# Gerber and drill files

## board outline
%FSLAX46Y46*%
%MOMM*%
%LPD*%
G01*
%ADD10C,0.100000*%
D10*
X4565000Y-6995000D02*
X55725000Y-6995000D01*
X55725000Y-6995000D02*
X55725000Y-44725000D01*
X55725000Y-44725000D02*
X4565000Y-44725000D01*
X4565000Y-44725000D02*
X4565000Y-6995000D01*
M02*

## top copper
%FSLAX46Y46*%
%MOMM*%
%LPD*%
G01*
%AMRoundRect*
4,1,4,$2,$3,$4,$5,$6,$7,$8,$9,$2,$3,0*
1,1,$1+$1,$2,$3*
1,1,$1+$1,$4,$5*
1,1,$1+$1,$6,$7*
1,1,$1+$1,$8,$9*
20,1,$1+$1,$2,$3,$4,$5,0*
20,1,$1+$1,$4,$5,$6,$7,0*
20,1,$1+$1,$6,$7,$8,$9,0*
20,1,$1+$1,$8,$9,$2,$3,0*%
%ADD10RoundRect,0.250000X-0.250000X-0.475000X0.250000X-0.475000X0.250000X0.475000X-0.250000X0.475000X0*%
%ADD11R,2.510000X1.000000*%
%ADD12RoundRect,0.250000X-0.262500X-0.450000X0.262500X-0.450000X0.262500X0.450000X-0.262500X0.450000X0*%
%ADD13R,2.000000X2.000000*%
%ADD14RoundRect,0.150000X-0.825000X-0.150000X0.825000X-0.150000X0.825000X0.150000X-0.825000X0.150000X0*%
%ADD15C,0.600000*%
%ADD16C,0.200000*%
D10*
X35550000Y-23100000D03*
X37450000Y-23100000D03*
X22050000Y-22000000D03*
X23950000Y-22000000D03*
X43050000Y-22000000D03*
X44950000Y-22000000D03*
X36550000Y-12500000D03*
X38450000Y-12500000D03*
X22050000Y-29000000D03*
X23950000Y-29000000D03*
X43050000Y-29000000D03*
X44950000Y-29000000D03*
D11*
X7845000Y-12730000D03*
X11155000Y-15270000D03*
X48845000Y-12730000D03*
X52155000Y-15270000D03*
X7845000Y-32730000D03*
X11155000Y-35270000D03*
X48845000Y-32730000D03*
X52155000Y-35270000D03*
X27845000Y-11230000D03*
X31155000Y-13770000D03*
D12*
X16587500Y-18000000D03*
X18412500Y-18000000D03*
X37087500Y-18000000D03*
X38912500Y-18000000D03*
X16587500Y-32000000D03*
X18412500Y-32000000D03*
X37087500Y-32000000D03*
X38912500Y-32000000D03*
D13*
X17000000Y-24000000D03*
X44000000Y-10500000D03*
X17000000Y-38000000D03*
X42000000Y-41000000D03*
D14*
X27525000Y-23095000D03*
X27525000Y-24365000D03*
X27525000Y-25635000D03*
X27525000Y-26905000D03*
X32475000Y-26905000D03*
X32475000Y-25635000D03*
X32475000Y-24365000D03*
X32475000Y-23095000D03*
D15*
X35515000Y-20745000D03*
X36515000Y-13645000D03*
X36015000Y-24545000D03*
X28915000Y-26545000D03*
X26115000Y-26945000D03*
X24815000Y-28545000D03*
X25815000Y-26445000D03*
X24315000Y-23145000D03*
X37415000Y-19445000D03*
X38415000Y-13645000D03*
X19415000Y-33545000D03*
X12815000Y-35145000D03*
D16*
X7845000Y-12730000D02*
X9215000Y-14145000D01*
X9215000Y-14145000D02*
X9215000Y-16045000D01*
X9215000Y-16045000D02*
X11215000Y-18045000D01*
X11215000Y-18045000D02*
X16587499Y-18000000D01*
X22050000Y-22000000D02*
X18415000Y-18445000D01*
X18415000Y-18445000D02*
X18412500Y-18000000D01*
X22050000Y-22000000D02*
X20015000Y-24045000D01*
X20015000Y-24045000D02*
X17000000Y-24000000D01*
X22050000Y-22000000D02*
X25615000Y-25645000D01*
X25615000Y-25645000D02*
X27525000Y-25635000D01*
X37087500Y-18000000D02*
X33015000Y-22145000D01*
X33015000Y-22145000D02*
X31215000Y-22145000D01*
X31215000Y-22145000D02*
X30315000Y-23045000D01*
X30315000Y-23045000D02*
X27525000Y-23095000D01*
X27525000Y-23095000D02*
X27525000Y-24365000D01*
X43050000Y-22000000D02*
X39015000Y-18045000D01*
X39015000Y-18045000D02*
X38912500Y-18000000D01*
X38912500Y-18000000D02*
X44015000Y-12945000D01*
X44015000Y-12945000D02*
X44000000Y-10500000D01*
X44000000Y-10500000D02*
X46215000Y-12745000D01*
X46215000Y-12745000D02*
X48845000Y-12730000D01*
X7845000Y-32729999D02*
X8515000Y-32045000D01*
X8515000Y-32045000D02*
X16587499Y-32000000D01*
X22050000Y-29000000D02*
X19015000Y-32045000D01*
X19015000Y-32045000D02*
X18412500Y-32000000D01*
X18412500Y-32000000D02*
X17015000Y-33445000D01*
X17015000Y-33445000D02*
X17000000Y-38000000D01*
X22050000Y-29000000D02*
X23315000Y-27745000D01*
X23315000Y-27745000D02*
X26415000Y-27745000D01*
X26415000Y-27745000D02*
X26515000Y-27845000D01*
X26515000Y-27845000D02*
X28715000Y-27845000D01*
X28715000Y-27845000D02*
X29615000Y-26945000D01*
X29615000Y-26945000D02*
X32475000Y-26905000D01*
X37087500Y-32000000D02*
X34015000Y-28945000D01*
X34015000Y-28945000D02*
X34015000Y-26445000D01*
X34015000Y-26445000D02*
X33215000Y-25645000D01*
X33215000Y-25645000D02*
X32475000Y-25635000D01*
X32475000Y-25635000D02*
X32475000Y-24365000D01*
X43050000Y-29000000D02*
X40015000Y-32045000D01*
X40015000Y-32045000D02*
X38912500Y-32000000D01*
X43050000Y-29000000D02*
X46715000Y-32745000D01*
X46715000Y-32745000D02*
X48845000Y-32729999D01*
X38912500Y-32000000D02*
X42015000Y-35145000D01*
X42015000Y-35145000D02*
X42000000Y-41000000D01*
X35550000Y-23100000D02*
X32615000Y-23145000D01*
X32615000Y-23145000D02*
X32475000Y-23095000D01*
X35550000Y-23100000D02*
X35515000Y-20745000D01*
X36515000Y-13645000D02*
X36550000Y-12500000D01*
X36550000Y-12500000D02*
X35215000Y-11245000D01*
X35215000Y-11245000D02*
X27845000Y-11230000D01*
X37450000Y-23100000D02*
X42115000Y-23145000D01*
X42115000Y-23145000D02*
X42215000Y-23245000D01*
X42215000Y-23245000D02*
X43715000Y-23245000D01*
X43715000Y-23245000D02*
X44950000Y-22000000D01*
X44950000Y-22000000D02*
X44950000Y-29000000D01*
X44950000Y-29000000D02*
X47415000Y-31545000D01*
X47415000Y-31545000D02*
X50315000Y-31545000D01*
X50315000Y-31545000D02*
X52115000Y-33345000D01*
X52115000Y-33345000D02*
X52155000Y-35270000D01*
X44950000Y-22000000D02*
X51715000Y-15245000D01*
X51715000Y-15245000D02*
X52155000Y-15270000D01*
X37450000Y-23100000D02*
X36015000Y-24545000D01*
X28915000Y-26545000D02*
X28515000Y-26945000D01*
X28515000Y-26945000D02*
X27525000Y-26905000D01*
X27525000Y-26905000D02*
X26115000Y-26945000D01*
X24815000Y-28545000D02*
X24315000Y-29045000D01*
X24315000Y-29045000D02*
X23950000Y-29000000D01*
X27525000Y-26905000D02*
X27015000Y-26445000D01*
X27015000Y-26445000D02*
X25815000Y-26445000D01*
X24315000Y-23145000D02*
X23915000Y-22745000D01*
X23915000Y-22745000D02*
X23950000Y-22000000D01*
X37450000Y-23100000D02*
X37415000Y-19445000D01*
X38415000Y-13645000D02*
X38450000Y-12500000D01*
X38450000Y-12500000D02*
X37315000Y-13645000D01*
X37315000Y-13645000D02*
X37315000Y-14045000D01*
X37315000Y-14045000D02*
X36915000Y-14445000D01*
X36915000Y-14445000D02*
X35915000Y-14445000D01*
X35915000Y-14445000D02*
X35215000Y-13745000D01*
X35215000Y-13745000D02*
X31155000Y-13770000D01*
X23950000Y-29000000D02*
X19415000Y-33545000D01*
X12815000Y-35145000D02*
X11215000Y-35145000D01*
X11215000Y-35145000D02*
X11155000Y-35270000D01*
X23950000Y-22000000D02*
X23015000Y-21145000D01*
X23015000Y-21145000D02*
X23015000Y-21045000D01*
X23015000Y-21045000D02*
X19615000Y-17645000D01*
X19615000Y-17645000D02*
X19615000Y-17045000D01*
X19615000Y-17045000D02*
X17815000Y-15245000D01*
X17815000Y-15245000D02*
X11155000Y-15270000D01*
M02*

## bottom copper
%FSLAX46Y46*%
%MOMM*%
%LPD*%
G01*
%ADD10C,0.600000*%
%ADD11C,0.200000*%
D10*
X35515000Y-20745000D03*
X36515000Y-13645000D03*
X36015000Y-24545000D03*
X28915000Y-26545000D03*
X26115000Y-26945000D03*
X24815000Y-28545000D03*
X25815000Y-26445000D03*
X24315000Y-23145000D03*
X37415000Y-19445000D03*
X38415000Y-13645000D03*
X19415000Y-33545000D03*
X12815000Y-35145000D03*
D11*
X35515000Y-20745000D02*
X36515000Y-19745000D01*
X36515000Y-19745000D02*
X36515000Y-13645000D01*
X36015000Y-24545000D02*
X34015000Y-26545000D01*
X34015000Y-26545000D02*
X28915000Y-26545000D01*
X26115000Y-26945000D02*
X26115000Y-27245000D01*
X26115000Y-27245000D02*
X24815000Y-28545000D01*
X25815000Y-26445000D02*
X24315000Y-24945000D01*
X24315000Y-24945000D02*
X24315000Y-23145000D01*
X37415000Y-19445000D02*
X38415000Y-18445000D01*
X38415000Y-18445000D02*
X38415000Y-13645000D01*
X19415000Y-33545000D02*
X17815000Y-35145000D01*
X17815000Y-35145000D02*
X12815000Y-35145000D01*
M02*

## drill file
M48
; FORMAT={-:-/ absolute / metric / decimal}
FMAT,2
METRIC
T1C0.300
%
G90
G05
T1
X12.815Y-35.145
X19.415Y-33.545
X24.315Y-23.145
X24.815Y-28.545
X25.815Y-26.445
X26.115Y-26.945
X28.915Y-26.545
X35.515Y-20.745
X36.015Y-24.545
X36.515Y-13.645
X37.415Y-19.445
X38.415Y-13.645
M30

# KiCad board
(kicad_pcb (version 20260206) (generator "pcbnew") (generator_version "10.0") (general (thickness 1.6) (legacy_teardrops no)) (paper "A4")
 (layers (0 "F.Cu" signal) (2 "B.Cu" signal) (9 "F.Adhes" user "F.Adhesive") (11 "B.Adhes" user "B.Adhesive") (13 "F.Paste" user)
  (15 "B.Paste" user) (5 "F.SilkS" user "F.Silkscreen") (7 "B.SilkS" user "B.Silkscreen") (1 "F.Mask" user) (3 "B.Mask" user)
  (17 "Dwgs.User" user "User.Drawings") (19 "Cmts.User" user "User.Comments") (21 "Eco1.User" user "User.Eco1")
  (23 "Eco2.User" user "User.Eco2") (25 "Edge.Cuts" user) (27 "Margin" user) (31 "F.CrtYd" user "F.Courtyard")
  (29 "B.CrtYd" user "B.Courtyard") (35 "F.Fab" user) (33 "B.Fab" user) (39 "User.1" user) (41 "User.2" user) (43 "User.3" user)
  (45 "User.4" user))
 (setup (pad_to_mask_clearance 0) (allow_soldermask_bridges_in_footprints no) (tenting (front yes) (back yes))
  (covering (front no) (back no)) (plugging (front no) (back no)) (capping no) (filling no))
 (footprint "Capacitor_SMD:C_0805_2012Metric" (layer "F.Cu") (at 36.5 23.1)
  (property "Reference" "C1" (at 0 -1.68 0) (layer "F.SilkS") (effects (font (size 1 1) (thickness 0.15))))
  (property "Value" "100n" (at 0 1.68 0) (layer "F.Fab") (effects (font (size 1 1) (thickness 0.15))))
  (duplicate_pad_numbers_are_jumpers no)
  (pad "1" smd roundrect (at -0.95 0) (size 1 1.45) (layers "F.Cu" "F.Mask" "F.Paste") (roundrect_rratio 0.25) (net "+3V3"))
  (pad "2" smd roundrect (at 0.95 0) (size 1 1.45) (layers "F.Cu" "F.Mask" "F.Paste") (roundrect_rratio 0.25) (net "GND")))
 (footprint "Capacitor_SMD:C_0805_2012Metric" (layer "F.Cu") (at 23 22)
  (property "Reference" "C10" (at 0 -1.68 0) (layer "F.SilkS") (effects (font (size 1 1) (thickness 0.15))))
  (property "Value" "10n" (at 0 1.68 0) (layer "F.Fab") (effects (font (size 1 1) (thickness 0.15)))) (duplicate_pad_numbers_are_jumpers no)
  (pad "1" smd roundrect (at -0.95 0) (size 1 1.45) (layers "F.Cu" "F.Mask" "F.Paste") (roundrect_rratio 0.25) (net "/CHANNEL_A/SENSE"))
  (pad "2" smd roundrect (at 0.95 0) (size 1 1.45) (layers "F.Cu" "F.Mask" "F.Paste") (roundrect_rratio 0.25) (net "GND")))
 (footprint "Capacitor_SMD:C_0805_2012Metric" (layer "F.Cu") (at 44 22)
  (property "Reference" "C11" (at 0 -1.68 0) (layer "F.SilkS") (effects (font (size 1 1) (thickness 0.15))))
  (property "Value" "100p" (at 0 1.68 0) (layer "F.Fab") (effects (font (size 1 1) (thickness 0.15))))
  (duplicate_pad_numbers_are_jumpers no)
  (pad "1" smd roundrect (at -0.95 0) (size 1 1.45) (layers "F.Cu" "F.Mask" "F.Paste") (roundrect_rratio 0.25) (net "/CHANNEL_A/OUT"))
  (pad "2" smd roundrect (at 0.95 0) (size 1 1.45) (layers "F.Cu" "F.Mask" "F.Paste") (roundrect_rratio 0.25) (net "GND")))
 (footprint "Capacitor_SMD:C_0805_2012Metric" (layer "F.Cu") (at 37.5 12.5)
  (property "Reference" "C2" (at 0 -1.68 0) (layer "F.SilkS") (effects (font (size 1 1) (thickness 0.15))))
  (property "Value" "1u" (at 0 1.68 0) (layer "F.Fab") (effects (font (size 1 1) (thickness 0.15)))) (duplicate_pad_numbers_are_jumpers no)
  (pad "1" smd roundrect (at -0.95 0) (size 1 1.45) (layers "F.Cu" "F.Mask" "F.Paste") (roundrect_rratio 0.25) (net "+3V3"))
  (pad "2" smd roundrect (at 0.95 0) (size 1 1.45) (layers "F.Cu" "F.Mask" "F.Paste") (roundrect_rratio 0.25) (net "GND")))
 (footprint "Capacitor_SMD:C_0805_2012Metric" (layer "F.Cu") (at 23 29)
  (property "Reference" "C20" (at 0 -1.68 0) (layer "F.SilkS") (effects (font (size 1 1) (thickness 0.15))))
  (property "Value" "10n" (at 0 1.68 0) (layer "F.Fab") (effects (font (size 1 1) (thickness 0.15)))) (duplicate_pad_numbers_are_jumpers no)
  (pad "1" smd roundrect (at -0.95 0) (size 1 1.45) (layers "F.Cu" "F.Mask" "F.Paste") (roundrect_rratio 0.25) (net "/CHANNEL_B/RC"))
  (pad "2" smd roundrect (at 0.95 0) (size 1 1.45) (layers "F.Cu" "F.Mask" "F.Paste") (roundrect_rratio 0.25) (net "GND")))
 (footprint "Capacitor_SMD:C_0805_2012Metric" (layer "F.Cu") (at 44 29)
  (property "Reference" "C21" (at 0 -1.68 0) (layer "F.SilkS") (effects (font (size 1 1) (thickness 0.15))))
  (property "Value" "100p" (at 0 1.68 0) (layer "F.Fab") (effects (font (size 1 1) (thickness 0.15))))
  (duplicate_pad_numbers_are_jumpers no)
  (pad "1" smd roundrect (at -0.95 0) (size 1 1.45) (layers "F.Cu" "F.Mask" "F.Paste") (roundrect_rratio 0.25) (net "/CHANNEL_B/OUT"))
  (pad "2" smd roundrect (at 0.95 0) (size 1 1.45) (layers "F.Cu" "F.Mask" "F.Paste") (roundrect_rratio 0.25) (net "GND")))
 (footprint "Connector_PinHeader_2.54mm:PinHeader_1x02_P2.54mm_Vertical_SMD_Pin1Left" (layer "F.Cu") (at 9.5 14)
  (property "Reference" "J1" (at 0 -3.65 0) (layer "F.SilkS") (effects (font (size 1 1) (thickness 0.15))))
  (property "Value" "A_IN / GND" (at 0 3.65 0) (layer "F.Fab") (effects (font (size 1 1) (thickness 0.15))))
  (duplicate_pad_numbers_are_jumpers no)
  (pad "1" smd rect (at -1.655 -1.27) (size 2.51 1) (layers "F.Cu" "F.Mask" "F.Paste") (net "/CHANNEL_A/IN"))
  (pad "2" smd rect (at 1.655 1.27) (size 2.51 1) (layers "F.Cu" "F.Mask" "F.Paste") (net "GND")))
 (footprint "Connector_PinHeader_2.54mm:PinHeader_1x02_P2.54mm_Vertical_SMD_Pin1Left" (layer "F.Cu") (at 50.5 14)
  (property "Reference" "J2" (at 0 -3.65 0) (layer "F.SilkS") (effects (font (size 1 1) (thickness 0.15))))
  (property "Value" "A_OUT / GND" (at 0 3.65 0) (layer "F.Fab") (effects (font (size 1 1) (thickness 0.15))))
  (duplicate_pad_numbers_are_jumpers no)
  (pad "1" smd rect (at -1.655 -1.27) (size 2.51 1) (layers "F.Cu" "F.Mask" "F.Paste") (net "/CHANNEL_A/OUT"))
  (pad "2" smd rect (at 1.655 1.27) (size 2.51 1) (layers "F.Cu" "F.Mask" "F.Paste") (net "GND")))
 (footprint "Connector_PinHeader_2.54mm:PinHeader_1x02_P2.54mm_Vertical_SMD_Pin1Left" (layer "F.Cu") (at 9.5 34)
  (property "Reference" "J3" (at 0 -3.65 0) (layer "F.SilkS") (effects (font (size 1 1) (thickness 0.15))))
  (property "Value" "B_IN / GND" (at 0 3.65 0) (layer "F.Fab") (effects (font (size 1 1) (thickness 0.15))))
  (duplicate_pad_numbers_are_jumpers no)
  (pad "1" smd rect (at -1.655 -1.27) (size 2.51 1) (layers "F.Cu" "F.Mask" "F.Paste") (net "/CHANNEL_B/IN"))
  (pad "2" smd rect (at 1.655 1.27) (size 2.51 1) (layers "F.Cu" "F.Mask" "F.Paste") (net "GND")))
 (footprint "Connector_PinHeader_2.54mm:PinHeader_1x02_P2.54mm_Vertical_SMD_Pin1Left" (layer "F.Cu") (at 50.5 34)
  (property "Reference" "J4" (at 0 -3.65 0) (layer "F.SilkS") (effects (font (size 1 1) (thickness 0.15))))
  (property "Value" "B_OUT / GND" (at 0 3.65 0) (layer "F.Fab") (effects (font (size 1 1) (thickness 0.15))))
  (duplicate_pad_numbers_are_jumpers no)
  (pad "1" smd rect (at -1.655 -1.27) (size 2.51 1) (layers "F.Cu" "F.Mask" "F.Paste") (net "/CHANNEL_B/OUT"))
  (pad "2" smd rect (at 1.655 1.27) (size 2.51 1) (layers "F.Cu" "F.Mask" "F.Paste") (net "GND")))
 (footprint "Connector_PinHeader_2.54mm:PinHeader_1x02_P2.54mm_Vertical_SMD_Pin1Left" (layer "F.Cu") (at 29.5 12.5)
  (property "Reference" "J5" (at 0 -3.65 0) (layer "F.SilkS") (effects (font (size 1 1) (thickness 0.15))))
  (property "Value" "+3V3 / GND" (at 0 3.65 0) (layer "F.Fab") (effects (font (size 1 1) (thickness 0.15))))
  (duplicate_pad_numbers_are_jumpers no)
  (pad "1" smd rect (at -1.655 -1.27) (size 2.51 1) (layers "F.Cu" "F.Mask" "F.Paste") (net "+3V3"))
  (pad "2" smd rect (at 1.655 1.27) (size 2.51 1) (layers "F.Cu" "F.Mask" "F.Paste") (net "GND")))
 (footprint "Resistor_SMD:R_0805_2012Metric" (layer "F.Cu") (at 17.5 18)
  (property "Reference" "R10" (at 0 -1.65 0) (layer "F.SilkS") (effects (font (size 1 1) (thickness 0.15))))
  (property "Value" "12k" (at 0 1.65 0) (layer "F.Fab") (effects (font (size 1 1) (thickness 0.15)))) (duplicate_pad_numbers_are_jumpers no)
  (pad "1" smd roundrect (at -0.9125 0) (size 1.025 1.4) (layers "F.Cu" "F.Mask" "F.Paste") (roundrect_rratio 0.243902)
   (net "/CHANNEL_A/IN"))
  (pad "2" smd roundrect (at 0.9125 0) (size 1.025 1.4) (layers "F.Cu" "F.Mask" "F.Paste") (roundrect_rratio 0.243902)
   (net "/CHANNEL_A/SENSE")))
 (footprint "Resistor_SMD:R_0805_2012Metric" (layer "F.Cu") (at 38 18)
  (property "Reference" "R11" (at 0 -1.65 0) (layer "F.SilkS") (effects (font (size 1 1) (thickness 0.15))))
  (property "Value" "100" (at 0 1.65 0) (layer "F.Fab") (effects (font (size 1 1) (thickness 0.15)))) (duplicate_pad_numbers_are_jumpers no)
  (pad "1" smd roundrect (at -0.9125 0) (size 1.025 1.4) (layers "F.Cu" "F.Mask" "F.Paste") (roundrect_rratio 0.243902)
   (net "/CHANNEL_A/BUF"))
  (pad "2" smd roundrect (at 0.9125 0) (size 1.025 1.4) (layers "F.Cu" "F.Mask" "F.Paste") (roundrect_rratio 0.243902)
   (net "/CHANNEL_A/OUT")))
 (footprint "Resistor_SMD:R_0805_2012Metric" (layer "F.Cu") (at 17.5 32)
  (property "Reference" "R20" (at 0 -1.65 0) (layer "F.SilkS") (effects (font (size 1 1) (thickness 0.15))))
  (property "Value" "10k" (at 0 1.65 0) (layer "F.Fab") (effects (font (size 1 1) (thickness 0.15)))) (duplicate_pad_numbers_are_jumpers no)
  (pad "1" smd roundrect (at -0.9125 0) (size 1.025 1.4) (layers "F.Cu" "F.Mask" "F.Paste") (roundrect_rratio 0.243902)
   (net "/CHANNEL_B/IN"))
  (pad "2" smd roundrect (at 0.9125 0) (size 1.025 1.4) (layers "F.Cu" "F.Mask" "F.Paste") (roundrect_rratio 0.243902) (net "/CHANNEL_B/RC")))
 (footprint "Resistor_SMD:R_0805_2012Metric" (layer "F.Cu") (at 38 32)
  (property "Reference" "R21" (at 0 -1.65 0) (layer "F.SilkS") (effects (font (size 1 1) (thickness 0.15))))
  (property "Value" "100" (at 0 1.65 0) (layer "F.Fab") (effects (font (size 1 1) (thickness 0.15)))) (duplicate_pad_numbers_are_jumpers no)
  (pad "1" smd roundrect (at -0.9125 0) (size 1.025 1.4) (layers "F.Cu" "F.Mask" "F.Paste") (roundrect_rratio 0.243902)
   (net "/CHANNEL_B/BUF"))
  (pad "2" smd roundrect (at 0.9125 0) (size 1.025 1.4) (layers "F.Cu" "F.Mask" "F.Paste") (roundrect_rratio 0.243902)
   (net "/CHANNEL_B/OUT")))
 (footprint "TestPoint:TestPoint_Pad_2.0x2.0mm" (layer "F.Cu") (at 17 24)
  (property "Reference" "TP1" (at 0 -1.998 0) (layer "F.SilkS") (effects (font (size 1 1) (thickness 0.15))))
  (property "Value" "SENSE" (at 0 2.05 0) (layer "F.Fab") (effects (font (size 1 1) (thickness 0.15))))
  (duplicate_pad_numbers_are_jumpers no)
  (pad "1" smd rect (at 0 0) (size 2 2) (layers "F.Cu" "F.Mask") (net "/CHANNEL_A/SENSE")))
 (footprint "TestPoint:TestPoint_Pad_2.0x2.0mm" (layer "F.Cu") (at 44 10.5)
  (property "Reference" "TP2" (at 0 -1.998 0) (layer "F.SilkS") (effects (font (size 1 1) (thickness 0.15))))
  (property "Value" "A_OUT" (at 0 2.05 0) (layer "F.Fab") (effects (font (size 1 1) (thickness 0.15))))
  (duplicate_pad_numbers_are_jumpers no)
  (pad "1" smd rect (at 0 0) (size 2 2) (layers "F.Cu" "F.Mask") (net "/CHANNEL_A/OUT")))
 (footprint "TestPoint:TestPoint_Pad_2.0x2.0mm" (layer "F.Cu") (at 17 38)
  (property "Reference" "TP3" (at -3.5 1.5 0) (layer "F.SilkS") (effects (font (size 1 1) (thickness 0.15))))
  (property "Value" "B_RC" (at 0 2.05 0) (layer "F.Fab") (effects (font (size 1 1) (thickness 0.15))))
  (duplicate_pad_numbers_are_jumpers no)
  (pad "1" smd rect (at 0 0) (size 2 2) (layers "F.Cu" "F.Mask") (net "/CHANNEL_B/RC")))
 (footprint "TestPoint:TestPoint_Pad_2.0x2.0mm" (layer "F.Cu") (at 42 41)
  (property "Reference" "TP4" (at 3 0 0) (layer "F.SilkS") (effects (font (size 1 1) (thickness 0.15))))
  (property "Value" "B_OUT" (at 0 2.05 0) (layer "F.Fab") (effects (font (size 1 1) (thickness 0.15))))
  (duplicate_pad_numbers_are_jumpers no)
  (pad "1" smd rect (at 0 0) (size 2 2) (layers "F.Cu" "F.Mask") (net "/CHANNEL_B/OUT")))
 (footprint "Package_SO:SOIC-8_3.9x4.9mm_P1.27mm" (layer "F.Cu") (at 30 25)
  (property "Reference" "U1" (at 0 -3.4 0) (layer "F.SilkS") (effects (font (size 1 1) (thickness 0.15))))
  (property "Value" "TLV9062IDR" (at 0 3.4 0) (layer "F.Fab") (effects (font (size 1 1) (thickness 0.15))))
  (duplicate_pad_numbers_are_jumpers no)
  (pad "1" smd roundrect (at -2.475 -1.905) (size 1.95 0.6) (layers "F.Cu" "F.Mask" "F.Paste") (roundrect_rratio 0.25)
   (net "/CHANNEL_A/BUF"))
  (pad "2" smd roundrect (at -2.475 -0.635) (size 1.95 0.6) (layers "F.Cu" "F.Mask" "F.Paste") (roundrect_rratio 0.25)
   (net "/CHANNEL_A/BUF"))
  (pad "3" smd roundrect (at -2.475 0.635) (size 1.95 0.6) (layers "F.Cu" "F.Mask" "F.Paste") (roundrect_rratio 0.25)
   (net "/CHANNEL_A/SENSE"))
  (pad "4" smd roundrect (at -2.475 1.905) (size 1.95 0.6) (layers "F.Cu" "F.Mask" "F.Paste") (roundrect_rratio 0.25) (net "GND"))
  (pad "5" smd roundrect (at 2.475 1.905) (size 1.95 0.6) (layers "F.Cu" "F.Mask" "F.Paste") (roundrect_rratio 0.25) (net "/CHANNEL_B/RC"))
  (pad "6" smd roundrect (at 2.475 0.635) (size 1.95 0.6) (layers "F.Cu" "F.Mask" "F.Paste") (roundrect_rratio 0.25) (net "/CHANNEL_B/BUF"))
  (pad "7" smd roundrect (at 2.475 -0.635) (size 1.95 0.6) (layers "F.Cu" "F.Mask" "F.Paste") (roundrect_rratio 0.25) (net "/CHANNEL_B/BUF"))
  (pad "8" smd roundrect (at 2.475 -1.905) (size 1.95 0.6) (layers "F.Cu" "F.Mask" "F.Paste") (roundrect_rratio 0.25) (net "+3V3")))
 (gr_line (start 4.565 6.995) (end 55.725 6.995) (stroke (width 0.1) (type default)) (layer "Edge.Cuts"))
 (gr_line (start 55.725 6.995) (end 55.725 44.725) (stroke (width 0.1) (type default)) (layer "Edge.Cuts"))
 (gr_line (start 55.725 44.725) (end 4.565 44.725) (stroke (width 0.1) (type default)) (layer "Edge.Cuts"))
 (gr_line (start 4.565 44.725) (end 4.565 6.995) (stroke (width 0.1) (type default)) (layer "Edge.Cuts"))
 (segment (start 7.845 12.73) (end 9.215 14.145) (width 0.2) (layer "F.Cu") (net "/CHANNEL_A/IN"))
 (segment (start 9.215 14.145) (end 9.215 16.045) (width 0.2) (layer "F.Cu") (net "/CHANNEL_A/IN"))
 (segment (start 9.215 16.045) (end 11.215 18.045) (width 0.2) (layer "F.Cu") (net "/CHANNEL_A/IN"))
 (segment (start 11.215 18.045) (end 16.587499 18) (width 0.2) (layer "F.Cu") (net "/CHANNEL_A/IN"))
 (segment (start 22.05 22) (end 18.415 18.445) (width 0.2) (layer "F.Cu") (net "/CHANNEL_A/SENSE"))
 (segment (start 18.415 18.445) (end 18.4125 18) (width 0.2) (layer "F.Cu") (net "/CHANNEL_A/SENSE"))
 (segment (start 22.05 22) (end 20.015 24.045) (width 0.2) (layer "F.Cu") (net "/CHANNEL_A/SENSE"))
 (segment (start 20.015 24.045) (end 17 24) (width 0.2) (layer "F.Cu") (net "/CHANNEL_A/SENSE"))
 (segment (start 22.05 22) (end 25.615 25.645) (width 0.2) (layer "F.Cu") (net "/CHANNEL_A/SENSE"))
 (segment (start 25.615 25.645) (end 27.525 25.635) (width 0.2) (layer "F.Cu") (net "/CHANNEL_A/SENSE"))
 (segment (start 37.0875 18) (end 33.015 22.145) (width 0.2) (layer "F.Cu") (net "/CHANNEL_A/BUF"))
 (segment (start 33.015 22.145) (end 31.215 22.145) (width 0.2) (layer "F.Cu") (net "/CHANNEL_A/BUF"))
 (segment (start 31.215 22.145) (end 30.315 23.045) (width 0.2) (layer "F.Cu") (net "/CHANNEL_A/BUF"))
 (segment (start 30.315 23.045) (end 27.525 23.095) (width 0.2) (layer "F.Cu") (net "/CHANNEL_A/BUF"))
 (segment (start 27.525 23.095) (end 27.525 24.365) (width 0.2) (layer "F.Cu") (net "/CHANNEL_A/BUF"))
 (segment (start 43.05 22) (end 39.015 18.045) (width 0.2) (layer "F.Cu") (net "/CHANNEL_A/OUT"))
 (segment (start 39.015 18.045) (end 38.9125 18) (width 0.2) (layer "F.Cu") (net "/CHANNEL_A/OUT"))
 (segment (start 38.9125 18) (end 44.015 12.945) (width 0.2) (layer "F.Cu") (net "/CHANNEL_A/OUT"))
 (segment (start 44.015 12.945) (end 44 10.5) (width 0.2) (layer "F.Cu") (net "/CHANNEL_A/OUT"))
 (segment (start 44 10.5) (end 46.215 12.745) (width 0.2) (layer "F.Cu") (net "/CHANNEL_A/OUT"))
 (segment (start 46.215 12.745) (end 48.845 12.73) (width 0.2) (layer "F.Cu") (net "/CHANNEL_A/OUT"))
 (segment (start 7.845 32.729999) (end 8.515 32.045) (width 0.2) (layer "F.Cu") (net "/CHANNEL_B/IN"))
 (segment (start 8.515 32.045) (end 16.587499 32) (width 0.2) (layer "F.Cu") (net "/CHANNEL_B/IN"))
 (segment (start 22.05 29) (end 19.015 32.045) (width 0.2) (layer "F.Cu") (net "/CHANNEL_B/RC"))
 (segment (start 19.015 32.045) (end 18.4125 32) (width 0.2) (layer "F.Cu") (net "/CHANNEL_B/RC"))
 (segment (start 18.4125 32) (end 17.015 33.445) (width 0.2) (layer "F.Cu") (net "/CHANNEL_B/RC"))
 (segment (start 17.015 33.445) (end 17 38) (width 0.2) (layer "F.Cu") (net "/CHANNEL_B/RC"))
 (segment (start 22.05 29) (end 23.315 27.745) (width 0.2) (layer "F.Cu") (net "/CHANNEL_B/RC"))
 (segment (start 23.315 27.745) (end 26.415 27.745) (width 0.2) (layer "F.Cu") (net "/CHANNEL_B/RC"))
 (segment (start 26.415 27.745) (end 26.515 27.845) (width 0.2) (layer "F.Cu") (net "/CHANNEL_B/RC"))
 (segment (start 26.515 27.845) (end 28.715 27.845) (width 0.2) (layer "F.Cu") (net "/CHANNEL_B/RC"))
 (segment (start 28.715 27.845) (end 29.615 26.945) (width 0.2) (layer "F.Cu") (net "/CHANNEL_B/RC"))
 (segment (start 29.615 26.945) (end 32.475 26.905) (width 0.2) (layer "F.Cu") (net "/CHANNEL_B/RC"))
 (segment (start 37.0875 32) (end 34.015 28.945) (width 0.2) (layer "F.Cu") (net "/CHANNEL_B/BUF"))
 (segment (start 34.015 28.945) (end 34.015 26.445) (width 0.2) (layer "F.Cu") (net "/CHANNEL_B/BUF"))
 (segment (start 34.015 26.445) (end 33.215 25.645) (width 0.2) (layer "F.Cu") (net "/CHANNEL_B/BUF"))
 (segment (start 33.215 25.645) (end 32.475 25.635) (width 0.2) (layer "F.Cu") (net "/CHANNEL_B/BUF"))
 (segment (start 32.475 25.635) (end 32.475 24.365) (width 0.2) (layer "F.Cu") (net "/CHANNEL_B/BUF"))
 (segment (start 43.05 29) (end 40.015 32.045) (width 0.2) (layer "F.Cu") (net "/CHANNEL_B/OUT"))
 (segment (start 40.015 32.045) (end 38.9125 32) (width 0.2) (layer "F.Cu") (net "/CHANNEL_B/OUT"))
 (segment (start 43.05 29) (end 46.715 32.745) (width 0.2) (layer "F.Cu") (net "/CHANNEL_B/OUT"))
 (segment (start 46.715 32.745) (end 48.845 32.729999) (width 0.2) (layer "F.Cu") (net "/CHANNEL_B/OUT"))
 (segment (start 38.9125 32) (end 42.015 35.145) (width 0.2) (layer "F.Cu") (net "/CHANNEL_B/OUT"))
 (segment (start 42.015 35.145) (end 42 41) (width 0.2) (layer "F.Cu") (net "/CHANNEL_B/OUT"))
 (segment (start 35.55 23.1) (end 32.615 23.145) (width 0.2) (layer "F.Cu") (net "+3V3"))
 (segment (start 32.615 23.145) (end 32.475 23.095) (width 0.2) (layer "F.Cu") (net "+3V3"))
 (segment (start 35.55 23.1) (end 35.515 20.745) (width 0.2) (layer "F.Cu") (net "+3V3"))
 (via (at 35.515 20.745) (size 0.6) (drill 0.3) (layers "F.Cu" "B.Cu") (capping no) (covering (front no) (back no))
  (plugging (front no) (back no)) (filling no) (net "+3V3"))
 (segment (start 35.515 20.745) (end 36.515 19.745) (width 0.2) (layer "B.Cu") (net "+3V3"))
 (segment (start 36.515 19.745) (end 36.515 13.645) (width 0.2) (layer "B.Cu") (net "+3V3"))
 (via (at 36.515 13.645) (size 0.6) (drill 0.3) (layers "F.Cu" "B.Cu") (capping no) (covering (front no) (back no))
  (plugging (front no) (back no)) (filling no) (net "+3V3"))
 (segment (start 36.515 13.645) (end 36.55 12.5) (width 0.2) (layer "F.Cu") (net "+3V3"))
 (segment (start 36.55 12.5) (end 35.215 11.245) (width 0.2) (layer "F.Cu") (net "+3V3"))
 (segment (start 35.215 11.245) (end 27.845 11.23) (width 0.2) (layer "F.Cu") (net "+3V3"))
 (segment (start 37.45 23.1) (end 42.115 23.145) (width 0.2) (layer "F.Cu") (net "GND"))
 (segment (start 42.115 23.145) (end 42.215 23.245) (width 0.2) (layer "F.Cu") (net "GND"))
 (segment (start 42.215 23.245) (end 43.715 23.245) (width 0.2) (layer "F.Cu") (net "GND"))
 (segment (start 43.715 23.245) (end 44.95 22) (width 0.2) (layer "F.Cu") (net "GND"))
 (segment (start 44.95 22) (end 44.95 29) (width 0.2) (layer "F.Cu") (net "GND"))
 (segment (start 44.95 29) (end 47.415 31.545) (width 0.2) (layer "F.Cu") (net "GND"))
 (segment (start 47.415 31.545) (end 50.315 31.545) (width 0.2) (layer "F.Cu") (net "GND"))
 (segment (start 50.315 31.545) (end 52.115 33.345) (width 0.2) (layer "F.Cu") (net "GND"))
 (segment (start 52.115 33.345) (end 52.155 35.27) (width 0.2) (layer "F.Cu") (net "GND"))
 (segment (start 44.95 22) (end 51.715 15.245) (width 0.2) (layer "F.Cu") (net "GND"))
 (segment (start 51.715 15.245) (end 52.155 15.27) (width 0.2) (layer "F.Cu") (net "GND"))
 (segment (start 37.45 23.1) (end 36.015 24.545) (width 0.2) (layer "F.Cu") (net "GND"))
 (via (at 36.015 24.545) (size 0.6) (drill 0.3) (layers "F.Cu" "B.Cu") (capping no) (covering (front no) (back no))
  (plugging (front no) (back no)) (filling no) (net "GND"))
 (segment (start 36.015 24.545) (end 34.015 26.545) (width 0.2) (layer "B.Cu") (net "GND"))
 (segment (start 34.015 26.545) (end 28.915 26.545) (width 0.2) (layer "B.Cu") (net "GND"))
 (via (at 28.915 26.545) (size 0.6) (drill 0.3) (layers "F.Cu" "B.Cu") (capping no) (covering (front no) (back no))
  (plugging (front no) (back no)) (filling no) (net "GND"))
 (segment (start 28.915 26.545) (end 28.515 26.945) (width 0.2) (layer "F.Cu") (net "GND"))
 (segment (start 28.515 26.945) (end 27.525 26.905) (width 0.2) (layer "F.Cu") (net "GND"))
 (segment (start 27.525 26.905) (end 26.115 26.945) (width 0.2) (layer "F.Cu") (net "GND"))
 (via (at 26.115 26.945) (size 0.6) (drill 0.3) (layers "F.Cu" "B.Cu") (capping no) (covering (front no) (back no))
  (plugging (front no) (back no)) (filling no) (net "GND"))
 (segment (start 26.115 26.945) (end 26.115 27.245) (width 0.2) (layer "B.Cu") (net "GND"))
 (segment (start 26.115 27.245) (end 24.815 28.545) (width 0.2) (layer "B.Cu") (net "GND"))
 (via (at 24.815 28.545) (size 0.6) (drill 0.3) (layers "F.Cu" "B.Cu") (capping no) (covering (front no) (back no))
  (plugging (front no) (back no)) (filling no) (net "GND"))
 (segment (start 24.815 28.545) (end 24.315 29.045) (width 0.2) (layer "F.Cu") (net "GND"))
 (segment (start 24.315 29.045) (end 23.95 29) (width 0.2) (layer "F.Cu") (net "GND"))
 (segment (start 27.525 26.905) (end 27.015 26.445) (width 0.2) (layer "F.Cu") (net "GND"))
 (segment (start 27.015 26.445) (end 25.815 26.445) (width 0.2) (layer "F.Cu") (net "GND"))
 (via (at 25.815 26.445) (size 0.6) (drill 0.3) (layers "F.Cu" "B.Cu") (capping no) (covering (front no) (back no))
  (plugging (front no) (back no)) (filling no) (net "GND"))
 (segment (start 25.815 26.445) (end 24.315 24.945) (width 0.2) (layer "B.Cu") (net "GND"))
 (segment (start 24.315 24.945) (end 24.315 23.145) (width 0.2) (layer "B.Cu") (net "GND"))
 (via (at 24.315 23.145) (size 0.6) (drill 0.3) (layers "F.Cu" "B.Cu") (capping no) (covering (front no) (back no))
  (plugging (front no) (back no)) (filling no) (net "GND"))
 (segment (start 24.315 23.145) (end 23.915 22.745) (width 0.2) (layer "F.Cu") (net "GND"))
 (segment (start 23.915 22.745) (end 23.95 22) (width 0.2) (layer "F.Cu") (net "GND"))
 (segment (start 37.45 23.1) (end 37.415 19.445) (width 0.2) (layer "F.Cu") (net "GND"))
 (via (at 37.415 19.445) (size 0.6) (drill 0.3) (layers "F.Cu" "B.Cu") (capping no) (covering (front no) (back no))
  (plugging (front no) (back no)) (filling no) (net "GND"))
 (segment (start 37.415 19.445) (end 38.415 18.445) (width 0.2) (layer "B.Cu") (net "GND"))
 (segment (start 38.415 18.445) (end 38.415 13.645) (width 0.2) (layer "B.Cu") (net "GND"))
 (via (at 38.415 13.645) (size 0.6) (drill 0.3) (layers "F.Cu" "B.Cu") (capping no) (covering (front no) (back no))
  (plugging (front no) (back no)) (filling no) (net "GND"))
 (segment (start 38.415 13.645) (end 38.45 12.5) (width 0.2) (layer "F.Cu") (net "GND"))
 (segment (start 38.45 12.5) (end 37.315 13.645) (width 0.2) (layer "F.Cu") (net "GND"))
 (segment (start 37.315 13.645) (end 37.315 14.045) (width 0.2) (layer "F.Cu") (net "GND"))
 (segment (start 37.315 14.045) (end 36.915 14.445) (width 0.2) (layer "F.Cu") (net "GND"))
 (segment (start 36.915 14.445) (end 35.915 14.445) (width 0.2) (layer "F.Cu") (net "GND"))
 (segment (start 35.915 14.445) (end 35.215 13.745) (width 0.2) (layer "F.Cu") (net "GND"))
 (segment (start 35.215 13.745) (end 31.155 13.77) (width 0.2) (layer "F.Cu") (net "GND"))
 (segment (start 23.95 29) (end 19.415 33.545) (width 0.2) (layer "F.Cu") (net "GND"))
 (via (at 19.415 33.545) (size 0.6) (drill 0.3) (layers "F.Cu" "B.Cu") (capping no) (covering (front no) (back no))
  (plugging (front no) (back no)) (filling no) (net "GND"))
 (segment (start 19.415 33.545) (end 17.815 35.145) (width 0.2) (layer "B.Cu") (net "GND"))
 (segment (start 17.815 35.145) (end 12.815 35.145) (width 0.2) (layer "B.Cu") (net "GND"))
 (via (at 12.815 35.145) (size 0.6) (drill 0.3) (layers "F.Cu" "B.Cu") (capping no) (covering (front no) (back no))
  (plugging (front no) (back no)) (filling no) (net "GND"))
 (segment (start 12.815 35.145) (end 11.215 35.145) (width 0.2) (layer "F.Cu") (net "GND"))
 (segment (start 11.215 35.145) (end 11.155 35.27) (width 0.2) (layer "F.Cu") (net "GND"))
 (segment (start 23.95 22) (end 23.015 21.145) (width 0.2) (layer "F.Cu") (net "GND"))
 (segment (start 23.015 21.145) (end 23.015 21.045) (width 0.2) (layer "F.Cu") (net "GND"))
 (segment (start 23.015 21.045) (end 19.615 17.645) (width 0.2) (layer "F.Cu") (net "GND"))
 (segment (start 19.615 17.645) (end 19.615 17.045) (width 0.2) (layer "F.Cu") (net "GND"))
 (segment (start 19.615 17.045) (end 17.815 15.245) (width 0.2) (layer "F.Cu") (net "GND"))
 (segment (start 17.815 15.245) (end 11.155 15.27) (width 0.2) (layer "F.Cu") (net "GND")))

